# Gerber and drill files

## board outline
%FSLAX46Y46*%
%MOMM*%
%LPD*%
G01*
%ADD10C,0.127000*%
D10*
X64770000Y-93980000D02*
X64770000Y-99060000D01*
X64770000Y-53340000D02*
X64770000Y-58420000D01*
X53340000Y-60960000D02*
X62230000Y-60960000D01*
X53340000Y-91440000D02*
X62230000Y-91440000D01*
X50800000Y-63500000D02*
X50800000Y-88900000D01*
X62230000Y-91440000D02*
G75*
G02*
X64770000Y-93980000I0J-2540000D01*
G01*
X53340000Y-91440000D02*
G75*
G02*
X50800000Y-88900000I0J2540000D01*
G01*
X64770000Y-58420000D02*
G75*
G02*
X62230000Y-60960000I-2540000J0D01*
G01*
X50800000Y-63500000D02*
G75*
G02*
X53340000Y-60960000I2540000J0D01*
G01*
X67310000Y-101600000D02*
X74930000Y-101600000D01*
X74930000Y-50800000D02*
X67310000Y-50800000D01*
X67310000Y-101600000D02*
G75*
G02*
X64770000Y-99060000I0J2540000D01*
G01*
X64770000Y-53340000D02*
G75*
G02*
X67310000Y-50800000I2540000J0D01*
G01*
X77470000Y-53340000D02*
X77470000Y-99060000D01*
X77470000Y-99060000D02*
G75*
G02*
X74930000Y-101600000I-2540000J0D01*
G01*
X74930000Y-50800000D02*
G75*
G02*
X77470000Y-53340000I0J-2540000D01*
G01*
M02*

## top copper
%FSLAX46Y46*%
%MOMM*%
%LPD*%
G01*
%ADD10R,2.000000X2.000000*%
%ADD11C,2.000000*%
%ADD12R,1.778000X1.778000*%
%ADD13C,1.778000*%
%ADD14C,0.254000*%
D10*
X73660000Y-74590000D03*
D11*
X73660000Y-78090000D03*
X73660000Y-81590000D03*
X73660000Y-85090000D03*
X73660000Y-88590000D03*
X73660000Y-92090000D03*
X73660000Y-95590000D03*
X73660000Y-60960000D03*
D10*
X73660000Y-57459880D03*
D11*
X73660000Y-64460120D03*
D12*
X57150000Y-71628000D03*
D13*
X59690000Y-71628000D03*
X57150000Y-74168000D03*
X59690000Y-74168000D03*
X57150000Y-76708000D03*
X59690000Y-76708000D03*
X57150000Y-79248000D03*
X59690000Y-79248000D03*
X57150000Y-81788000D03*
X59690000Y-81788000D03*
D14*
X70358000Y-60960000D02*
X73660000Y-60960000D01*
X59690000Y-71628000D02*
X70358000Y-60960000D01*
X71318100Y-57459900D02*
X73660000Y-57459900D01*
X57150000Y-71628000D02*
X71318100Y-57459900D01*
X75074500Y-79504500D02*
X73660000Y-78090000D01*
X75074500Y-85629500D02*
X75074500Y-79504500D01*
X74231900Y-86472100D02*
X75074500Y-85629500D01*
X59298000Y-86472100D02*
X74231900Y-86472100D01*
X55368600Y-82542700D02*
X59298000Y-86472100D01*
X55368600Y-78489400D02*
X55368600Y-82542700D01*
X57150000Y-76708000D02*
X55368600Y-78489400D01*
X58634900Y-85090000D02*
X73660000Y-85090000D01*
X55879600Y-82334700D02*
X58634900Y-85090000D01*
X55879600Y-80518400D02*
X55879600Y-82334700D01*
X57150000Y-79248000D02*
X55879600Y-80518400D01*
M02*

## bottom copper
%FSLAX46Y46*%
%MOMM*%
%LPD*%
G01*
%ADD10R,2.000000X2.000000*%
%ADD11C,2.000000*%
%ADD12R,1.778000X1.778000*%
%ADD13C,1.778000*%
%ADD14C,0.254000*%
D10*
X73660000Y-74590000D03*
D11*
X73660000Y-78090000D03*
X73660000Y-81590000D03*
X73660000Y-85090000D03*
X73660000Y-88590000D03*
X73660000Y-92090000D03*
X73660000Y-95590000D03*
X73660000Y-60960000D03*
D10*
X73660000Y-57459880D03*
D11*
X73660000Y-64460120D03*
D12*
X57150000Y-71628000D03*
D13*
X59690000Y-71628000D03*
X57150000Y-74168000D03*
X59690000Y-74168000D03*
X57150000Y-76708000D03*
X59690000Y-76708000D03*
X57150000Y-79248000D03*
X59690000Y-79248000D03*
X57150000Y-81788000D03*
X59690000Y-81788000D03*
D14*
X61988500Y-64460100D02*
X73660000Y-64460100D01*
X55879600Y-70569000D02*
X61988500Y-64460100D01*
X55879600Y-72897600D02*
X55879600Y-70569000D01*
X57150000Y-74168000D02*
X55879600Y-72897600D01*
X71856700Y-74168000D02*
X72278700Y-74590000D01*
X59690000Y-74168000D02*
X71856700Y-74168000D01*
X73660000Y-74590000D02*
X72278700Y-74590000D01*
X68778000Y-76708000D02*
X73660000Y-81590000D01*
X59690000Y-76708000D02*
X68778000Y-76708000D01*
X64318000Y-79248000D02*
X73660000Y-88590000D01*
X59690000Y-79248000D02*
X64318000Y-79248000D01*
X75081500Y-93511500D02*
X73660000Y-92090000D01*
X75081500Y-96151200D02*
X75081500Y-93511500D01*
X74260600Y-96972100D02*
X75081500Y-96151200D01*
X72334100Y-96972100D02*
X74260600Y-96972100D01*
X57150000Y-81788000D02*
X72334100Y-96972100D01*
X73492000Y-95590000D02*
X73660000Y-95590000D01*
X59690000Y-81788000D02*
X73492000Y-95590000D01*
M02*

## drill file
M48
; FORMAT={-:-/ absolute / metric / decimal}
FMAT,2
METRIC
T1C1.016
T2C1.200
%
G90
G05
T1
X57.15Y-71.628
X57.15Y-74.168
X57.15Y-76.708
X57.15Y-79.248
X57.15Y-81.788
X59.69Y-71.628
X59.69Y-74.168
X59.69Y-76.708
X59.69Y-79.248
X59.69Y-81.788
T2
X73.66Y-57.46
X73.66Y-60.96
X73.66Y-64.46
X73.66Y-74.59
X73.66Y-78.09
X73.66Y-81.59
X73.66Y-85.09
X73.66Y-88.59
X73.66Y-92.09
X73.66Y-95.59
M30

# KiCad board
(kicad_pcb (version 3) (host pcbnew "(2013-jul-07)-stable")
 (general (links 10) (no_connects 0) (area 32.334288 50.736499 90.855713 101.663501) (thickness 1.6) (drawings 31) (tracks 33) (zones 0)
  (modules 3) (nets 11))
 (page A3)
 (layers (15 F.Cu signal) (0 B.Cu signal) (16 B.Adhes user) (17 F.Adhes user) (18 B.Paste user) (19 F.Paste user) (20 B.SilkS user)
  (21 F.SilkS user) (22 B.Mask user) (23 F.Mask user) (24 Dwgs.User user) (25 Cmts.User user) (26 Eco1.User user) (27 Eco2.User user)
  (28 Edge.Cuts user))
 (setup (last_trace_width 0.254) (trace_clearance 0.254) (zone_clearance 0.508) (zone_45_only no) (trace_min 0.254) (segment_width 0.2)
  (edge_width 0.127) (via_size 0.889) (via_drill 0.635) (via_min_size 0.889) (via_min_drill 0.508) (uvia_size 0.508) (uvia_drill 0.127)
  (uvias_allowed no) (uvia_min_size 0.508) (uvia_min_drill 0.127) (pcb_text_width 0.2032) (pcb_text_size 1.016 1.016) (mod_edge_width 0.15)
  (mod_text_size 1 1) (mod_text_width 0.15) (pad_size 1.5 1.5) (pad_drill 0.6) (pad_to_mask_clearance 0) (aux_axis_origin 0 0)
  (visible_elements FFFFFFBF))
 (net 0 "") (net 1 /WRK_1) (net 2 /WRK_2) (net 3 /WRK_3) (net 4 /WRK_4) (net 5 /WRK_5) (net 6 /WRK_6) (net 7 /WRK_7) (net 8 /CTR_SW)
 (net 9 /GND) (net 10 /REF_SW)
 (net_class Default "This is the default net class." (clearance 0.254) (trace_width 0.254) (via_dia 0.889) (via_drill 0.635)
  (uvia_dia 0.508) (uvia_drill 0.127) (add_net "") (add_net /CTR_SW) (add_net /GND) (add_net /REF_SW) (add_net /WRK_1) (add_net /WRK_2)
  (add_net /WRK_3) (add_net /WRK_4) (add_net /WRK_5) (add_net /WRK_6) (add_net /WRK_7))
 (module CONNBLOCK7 (layer F.Cu) (at 73.66 85.09 270)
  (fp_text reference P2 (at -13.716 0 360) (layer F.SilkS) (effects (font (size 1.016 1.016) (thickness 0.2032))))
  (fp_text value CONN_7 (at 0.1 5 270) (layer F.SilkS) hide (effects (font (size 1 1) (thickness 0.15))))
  (pad 1 thru_hole rect (at -10.5 0 270) (size 2 2) (drill 1.2) (layers *.Cu *.Mask F.SilkS) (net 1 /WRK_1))
  (pad 2 thru_hole circle (at -7 0 270) (size 2 2) (drill 1.2) (layers *.Cu *.Mask F.SilkS) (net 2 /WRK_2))
  (pad 3 thru_hole circle (at -3.5 0 270) (size 2 2) (drill 1.2) (layers *.Cu *.Mask F.SilkS) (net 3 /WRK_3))
  (pad 4 thru_hole circle (at 0 0 270) (size 2 2) (drill 1.2) (layers *.Cu *.Mask F.SilkS) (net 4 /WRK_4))
  (pad 5 thru_hole circle (at 3.5 0 270) (size 2 2) (drill 1.2) (layers *.Cu *.Mask F.SilkS) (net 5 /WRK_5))
  (pad 6 thru_hole circle (at 7 0 270) (size 2 2) (drill 1.2) (layers *.Cu *.Mask F.SilkS) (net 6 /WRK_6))
  (pad 7 thru_hole circle (at 10.5 0 270) (size 2 2) (drill 1.2) (layers *.Cu *.Mask F.SilkS) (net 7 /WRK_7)))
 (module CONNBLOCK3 (layer F.Cu) (at 73.66 60.96 270)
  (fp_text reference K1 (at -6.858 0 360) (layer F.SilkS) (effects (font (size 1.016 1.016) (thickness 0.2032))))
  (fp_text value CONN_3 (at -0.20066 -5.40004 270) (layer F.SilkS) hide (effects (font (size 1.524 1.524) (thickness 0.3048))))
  (pad 2 thru_hole circle (at 0 0 270) (size 2 2) (drill 1.2) (layers *.Cu *.Mask F.SilkS) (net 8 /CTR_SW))
  (pad 1 thru_hole rect (at -3.50012 0 270) (size 2 2) (drill 1.2) (layers *.Cu *.Mask F.SilkS) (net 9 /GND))
  (pad 3 thru_hole circle (at 3.50012 0 270) (size 2 2) (drill 1.2) (layers *.Cu *.Mask F.SilkS) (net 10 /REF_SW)))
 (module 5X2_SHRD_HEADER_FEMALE (layer B.Cu) (at 58.42 76.2 90)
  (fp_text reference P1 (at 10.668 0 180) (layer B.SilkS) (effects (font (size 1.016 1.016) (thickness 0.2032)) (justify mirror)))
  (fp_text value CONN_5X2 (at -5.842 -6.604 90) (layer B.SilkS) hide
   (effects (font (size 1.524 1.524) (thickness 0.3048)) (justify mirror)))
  (pad 1 thru_hole rect (at 4.572 -1.27 270) (size 1.778 1.778) (drill 1.016) (layers *.Cu *.Mask B.SilkS) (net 9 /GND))
  (pad 2 thru_hole circle (at 4.572 1.27 270) (size 1.778 1.778) (drill 1.016) (layers *.Cu *.Mask B.SilkS) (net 8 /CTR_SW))
  (pad 3 thru_hole circle (at 2.032 -1.27 270) (size 1.778 1.778) (drill 1.016) (layers *.Cu *.Mask B.SilkS) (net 10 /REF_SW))
  (pad 4 thru_hole circle (at 2.032 1.27 270) (size 1.778 1.778) (drill 1.016) (layers *.Cu *.Mask B.SilkS) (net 1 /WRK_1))
  (pad 5 thru_hole circle (at -0.508 -1.27 270) (size 1.778 1.778) (drill 1.016) (layers *.Cu *.Mask B.SilkS) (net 2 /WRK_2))
  (pad 6 thru_hole circle (at -0.508 1.27 270) (size 1.778 1.778) (drill 1.016) (layers *.Cu *.Mask B.SilkS) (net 3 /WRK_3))
  (pad 7 thru_hole circle (at -3.048 -1.27 270) (size 1.778 1.778) (drill 1.016) (layers *.Cu *.Mask B.SilkS) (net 4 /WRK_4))
  (pad 8 thru_hole circle (at -3.048 1.27 270) (size 1.778 1.778) (drill 1.016) (layers *.Cu *.Mask B.SilkS) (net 5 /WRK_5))
  (pad 9 thru_hole circle (at -5.588 -1.27 270) (size 1.778 1.778) (drill 1.016) (layers *.Cu *.Mask B.SilkS) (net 6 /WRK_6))
  (pad 10 thru_hole circle (at -5.588 1.27 270) (size 1.778 1.778) (drill 1.016) (layers *.Cu *.Mask B.SilkS) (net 7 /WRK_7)))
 (gr_line (start 64.77 93.98) (end 64.77 99.06) (angle 90) (layer Edge.Cuts) (width 0.127))
 (gr_line (start 64.77 53.34) (end 64.77 58.42) (angle 90) (layer Edge.Cuts) (width 0.127))
 (gr_line (start 53.34 60.96) (end 62.23 60.96) (angle 90) (layer Edge.Cuts) (width 0.127))
 (gr_line (start 53.34 91.44) (end 62.23 91.44) (angle 90) (layer Edge.Cuts) (width 0.127))
 (gr_line (start 50.8 63.5) (end 50.8 88.9) (angle 90) (layer Edge.Cuts) (width 0.127))
 (gr_arc (start 62.23 93.98) (end 62.23 91.44) (angle 90) (layer Edge.Cuts) (width 0.127))
 (gr_arc (start 53.34 88.9) (end 53.34 91.44) (angle 90) (layer Edge.Cuts) (width 0.127))
 (gr_arc (start 62.23 58.42) (end 64.77 58.42) (angle 90) (layer Edge.Cuts) (width 0.127))
 (gr_arc (start 53.34 63.5) (end 50.8 63.5) (angle 90) (layer Edge.Cuts) (width 0.127))
 (gr_line (start 67.31 101.6) (end 74.93 101.6) (angle 90) (layer Edge.Cuts) (width 0.127))
 (gr_line (start 74.93 50.8) (end 67.31 50.8) (angle 90) (layer Edge.Cuts) (width 0.127))
 (gr_arc (start 67.31 99.06) (end 67.31 101.6) (angle 90) (layer Edge.Cuts) (width 0.127))
 (gr_arc (start 67.31 53.34) (end 64.77 53.34) (angle 90) (layer Edge.Cuts) (width 0.127))
 (gr_line (start 77.47 53.34) (end 77.47 99.06) (angle 90) (layer Edge.Cuts) (width 0.127))
 (gr_arc (start 74.93 99.06) (end 77.47 99.06) (angle 90) (layer Edge.Cuts) (width 0.127))
 (gr_arc (start 74.93 53.34) (end 74.93 50.8) (angle 90) (layer Edge.Cuts) (width 0.127))
 (segment (start 70.358 60.96) (end 73.66 60.96) (width 0.254) (layer F.Cu) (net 8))
 (segment (start 59.69 71.628) (end 70.358 60.96) (width 0.254) (layer F.Cu) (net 8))
 (segment (start 71.3181 57.4599) (end 73.66 57.4599) (width 0.254) (layer F.Cu) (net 9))
 (segment (start 57.15 71.628) (end 71.3181 57.4599) (width 0.254) (layer F.Cu) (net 9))
 (segment (start 61.9885 64.4601) (end 73.66 64.4601) (width 0.254) (layer B.Cu) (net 10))
 (segment (start 55.8796 70.569) (end 61.9885 64.4601) (width 0.254) (layer B.Cu) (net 10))
 (segment (start 55.8796 72.8976) (end 55.8796 70.569) (width 0.254) (layer B.Cu) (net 10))
 (segment (start 57.15 74.168) (end 55.8796 72.8976) (width 0.254) (layer B.Cu) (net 10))
 (segment (start 71.8567 74.168) (end 72.2787 74.59) (width 0.254) (layer B.Cu) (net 1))
 (segment (start 59.69 74.168) (end 71.8567 74.168) (width 0.254) (layer B.Cu) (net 1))
 (segment (start 73.66 74.59) (end 72.2787 74.59) (width 0.254) (layer B.Cu) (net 1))
 (segment (start 75.0745 79.5045) (end 73.66 78.09) (width 0.254) (layer F.Cu) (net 2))
 (segment (start 75.0745 85.6295) (end 75.0745 79.5045) (width 0.254) (layer F.Cu) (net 2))
 (segment (start 74.2319 86.4721) (end 75.0745 85.6295) (width 0.254) (layer F.Cu) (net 2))
 (segment (start 59.298 86.4721) (end 74.2319 86.4721) (width 0.254) (layer F.Cu) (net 2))
 (segment (start 55.3686 82.5427) (end 59.298 86.4721) (width 0.254) (layer F.Cu) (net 2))
 (segment (start 55.3686 78.4894) (end 55.3686 82.5427) (width 0.254) (layer F.Cu) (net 2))
 (segment (start 57.15 76.708) (end 55.3686 78.4894) (width 0.254) (layer F.Cu) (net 2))
 (segment (start 68.778 76.708) (end 73.66 81.59) (width 0.254) (layer B.Cu) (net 3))
 (segment (start 59.69 76.708) (end 68.778 76.708) (width 0.254) (layer B.Cu) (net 3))
 (segment (start 58.6349 85.09) (end 73.66 85.09) (width 0.254) (layer F.Cu) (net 4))
 (segment (start 55.8796 82.3347) (end 58.6349 85.09) (width 0.254) (layer F.Cu) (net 4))
 (segment (start 55.8796 80.5184) (end 55.8796 82.3347) (width 0.254) (layer F.Cu) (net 4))
 (segment (start 57.15 79.248) (end 55.8796 80.5184) (width 0.254) (layer F.Cu) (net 4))
 (segment (start 64.318 79.248) (end 73.66 88.59) (width 0.254) (layer B.Cu) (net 5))
 (segment (start 59.69 79.248) (end 64.318 79.248) (width 0.254) (layer B.Cu) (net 5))
 (segment (start 75.0815 93.5115) (end 73.66 92.09) (width 0.254) (layer B.Cu) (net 6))
 (segment (start 75.0815 96.1512) (end 75.0815 93.5115) (width 0.254) (layer B.Cu) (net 6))
 (segment (start 74.2606 96.9721) (end 75.0815 96.1512) (width 0.254) (layer B.Cu) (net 6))
 (segment (start 72.3341 96.9721) (end 74.2606 96.9721) (width 0.254) (layer B.Cu) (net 6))
 (segment (start 57.15 81.788) (end 72.3341 96.9721) (width 0.254) (layer B.Cu) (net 6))
 (segment (start 73.492 95.59) (end 73.66 95.59) (width 0.254) (layer B.Cu) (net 7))
 (segment (start 59.69 81.788) (end 73.492 95.59) (width 0.254) (layer B.Cu) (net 7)))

